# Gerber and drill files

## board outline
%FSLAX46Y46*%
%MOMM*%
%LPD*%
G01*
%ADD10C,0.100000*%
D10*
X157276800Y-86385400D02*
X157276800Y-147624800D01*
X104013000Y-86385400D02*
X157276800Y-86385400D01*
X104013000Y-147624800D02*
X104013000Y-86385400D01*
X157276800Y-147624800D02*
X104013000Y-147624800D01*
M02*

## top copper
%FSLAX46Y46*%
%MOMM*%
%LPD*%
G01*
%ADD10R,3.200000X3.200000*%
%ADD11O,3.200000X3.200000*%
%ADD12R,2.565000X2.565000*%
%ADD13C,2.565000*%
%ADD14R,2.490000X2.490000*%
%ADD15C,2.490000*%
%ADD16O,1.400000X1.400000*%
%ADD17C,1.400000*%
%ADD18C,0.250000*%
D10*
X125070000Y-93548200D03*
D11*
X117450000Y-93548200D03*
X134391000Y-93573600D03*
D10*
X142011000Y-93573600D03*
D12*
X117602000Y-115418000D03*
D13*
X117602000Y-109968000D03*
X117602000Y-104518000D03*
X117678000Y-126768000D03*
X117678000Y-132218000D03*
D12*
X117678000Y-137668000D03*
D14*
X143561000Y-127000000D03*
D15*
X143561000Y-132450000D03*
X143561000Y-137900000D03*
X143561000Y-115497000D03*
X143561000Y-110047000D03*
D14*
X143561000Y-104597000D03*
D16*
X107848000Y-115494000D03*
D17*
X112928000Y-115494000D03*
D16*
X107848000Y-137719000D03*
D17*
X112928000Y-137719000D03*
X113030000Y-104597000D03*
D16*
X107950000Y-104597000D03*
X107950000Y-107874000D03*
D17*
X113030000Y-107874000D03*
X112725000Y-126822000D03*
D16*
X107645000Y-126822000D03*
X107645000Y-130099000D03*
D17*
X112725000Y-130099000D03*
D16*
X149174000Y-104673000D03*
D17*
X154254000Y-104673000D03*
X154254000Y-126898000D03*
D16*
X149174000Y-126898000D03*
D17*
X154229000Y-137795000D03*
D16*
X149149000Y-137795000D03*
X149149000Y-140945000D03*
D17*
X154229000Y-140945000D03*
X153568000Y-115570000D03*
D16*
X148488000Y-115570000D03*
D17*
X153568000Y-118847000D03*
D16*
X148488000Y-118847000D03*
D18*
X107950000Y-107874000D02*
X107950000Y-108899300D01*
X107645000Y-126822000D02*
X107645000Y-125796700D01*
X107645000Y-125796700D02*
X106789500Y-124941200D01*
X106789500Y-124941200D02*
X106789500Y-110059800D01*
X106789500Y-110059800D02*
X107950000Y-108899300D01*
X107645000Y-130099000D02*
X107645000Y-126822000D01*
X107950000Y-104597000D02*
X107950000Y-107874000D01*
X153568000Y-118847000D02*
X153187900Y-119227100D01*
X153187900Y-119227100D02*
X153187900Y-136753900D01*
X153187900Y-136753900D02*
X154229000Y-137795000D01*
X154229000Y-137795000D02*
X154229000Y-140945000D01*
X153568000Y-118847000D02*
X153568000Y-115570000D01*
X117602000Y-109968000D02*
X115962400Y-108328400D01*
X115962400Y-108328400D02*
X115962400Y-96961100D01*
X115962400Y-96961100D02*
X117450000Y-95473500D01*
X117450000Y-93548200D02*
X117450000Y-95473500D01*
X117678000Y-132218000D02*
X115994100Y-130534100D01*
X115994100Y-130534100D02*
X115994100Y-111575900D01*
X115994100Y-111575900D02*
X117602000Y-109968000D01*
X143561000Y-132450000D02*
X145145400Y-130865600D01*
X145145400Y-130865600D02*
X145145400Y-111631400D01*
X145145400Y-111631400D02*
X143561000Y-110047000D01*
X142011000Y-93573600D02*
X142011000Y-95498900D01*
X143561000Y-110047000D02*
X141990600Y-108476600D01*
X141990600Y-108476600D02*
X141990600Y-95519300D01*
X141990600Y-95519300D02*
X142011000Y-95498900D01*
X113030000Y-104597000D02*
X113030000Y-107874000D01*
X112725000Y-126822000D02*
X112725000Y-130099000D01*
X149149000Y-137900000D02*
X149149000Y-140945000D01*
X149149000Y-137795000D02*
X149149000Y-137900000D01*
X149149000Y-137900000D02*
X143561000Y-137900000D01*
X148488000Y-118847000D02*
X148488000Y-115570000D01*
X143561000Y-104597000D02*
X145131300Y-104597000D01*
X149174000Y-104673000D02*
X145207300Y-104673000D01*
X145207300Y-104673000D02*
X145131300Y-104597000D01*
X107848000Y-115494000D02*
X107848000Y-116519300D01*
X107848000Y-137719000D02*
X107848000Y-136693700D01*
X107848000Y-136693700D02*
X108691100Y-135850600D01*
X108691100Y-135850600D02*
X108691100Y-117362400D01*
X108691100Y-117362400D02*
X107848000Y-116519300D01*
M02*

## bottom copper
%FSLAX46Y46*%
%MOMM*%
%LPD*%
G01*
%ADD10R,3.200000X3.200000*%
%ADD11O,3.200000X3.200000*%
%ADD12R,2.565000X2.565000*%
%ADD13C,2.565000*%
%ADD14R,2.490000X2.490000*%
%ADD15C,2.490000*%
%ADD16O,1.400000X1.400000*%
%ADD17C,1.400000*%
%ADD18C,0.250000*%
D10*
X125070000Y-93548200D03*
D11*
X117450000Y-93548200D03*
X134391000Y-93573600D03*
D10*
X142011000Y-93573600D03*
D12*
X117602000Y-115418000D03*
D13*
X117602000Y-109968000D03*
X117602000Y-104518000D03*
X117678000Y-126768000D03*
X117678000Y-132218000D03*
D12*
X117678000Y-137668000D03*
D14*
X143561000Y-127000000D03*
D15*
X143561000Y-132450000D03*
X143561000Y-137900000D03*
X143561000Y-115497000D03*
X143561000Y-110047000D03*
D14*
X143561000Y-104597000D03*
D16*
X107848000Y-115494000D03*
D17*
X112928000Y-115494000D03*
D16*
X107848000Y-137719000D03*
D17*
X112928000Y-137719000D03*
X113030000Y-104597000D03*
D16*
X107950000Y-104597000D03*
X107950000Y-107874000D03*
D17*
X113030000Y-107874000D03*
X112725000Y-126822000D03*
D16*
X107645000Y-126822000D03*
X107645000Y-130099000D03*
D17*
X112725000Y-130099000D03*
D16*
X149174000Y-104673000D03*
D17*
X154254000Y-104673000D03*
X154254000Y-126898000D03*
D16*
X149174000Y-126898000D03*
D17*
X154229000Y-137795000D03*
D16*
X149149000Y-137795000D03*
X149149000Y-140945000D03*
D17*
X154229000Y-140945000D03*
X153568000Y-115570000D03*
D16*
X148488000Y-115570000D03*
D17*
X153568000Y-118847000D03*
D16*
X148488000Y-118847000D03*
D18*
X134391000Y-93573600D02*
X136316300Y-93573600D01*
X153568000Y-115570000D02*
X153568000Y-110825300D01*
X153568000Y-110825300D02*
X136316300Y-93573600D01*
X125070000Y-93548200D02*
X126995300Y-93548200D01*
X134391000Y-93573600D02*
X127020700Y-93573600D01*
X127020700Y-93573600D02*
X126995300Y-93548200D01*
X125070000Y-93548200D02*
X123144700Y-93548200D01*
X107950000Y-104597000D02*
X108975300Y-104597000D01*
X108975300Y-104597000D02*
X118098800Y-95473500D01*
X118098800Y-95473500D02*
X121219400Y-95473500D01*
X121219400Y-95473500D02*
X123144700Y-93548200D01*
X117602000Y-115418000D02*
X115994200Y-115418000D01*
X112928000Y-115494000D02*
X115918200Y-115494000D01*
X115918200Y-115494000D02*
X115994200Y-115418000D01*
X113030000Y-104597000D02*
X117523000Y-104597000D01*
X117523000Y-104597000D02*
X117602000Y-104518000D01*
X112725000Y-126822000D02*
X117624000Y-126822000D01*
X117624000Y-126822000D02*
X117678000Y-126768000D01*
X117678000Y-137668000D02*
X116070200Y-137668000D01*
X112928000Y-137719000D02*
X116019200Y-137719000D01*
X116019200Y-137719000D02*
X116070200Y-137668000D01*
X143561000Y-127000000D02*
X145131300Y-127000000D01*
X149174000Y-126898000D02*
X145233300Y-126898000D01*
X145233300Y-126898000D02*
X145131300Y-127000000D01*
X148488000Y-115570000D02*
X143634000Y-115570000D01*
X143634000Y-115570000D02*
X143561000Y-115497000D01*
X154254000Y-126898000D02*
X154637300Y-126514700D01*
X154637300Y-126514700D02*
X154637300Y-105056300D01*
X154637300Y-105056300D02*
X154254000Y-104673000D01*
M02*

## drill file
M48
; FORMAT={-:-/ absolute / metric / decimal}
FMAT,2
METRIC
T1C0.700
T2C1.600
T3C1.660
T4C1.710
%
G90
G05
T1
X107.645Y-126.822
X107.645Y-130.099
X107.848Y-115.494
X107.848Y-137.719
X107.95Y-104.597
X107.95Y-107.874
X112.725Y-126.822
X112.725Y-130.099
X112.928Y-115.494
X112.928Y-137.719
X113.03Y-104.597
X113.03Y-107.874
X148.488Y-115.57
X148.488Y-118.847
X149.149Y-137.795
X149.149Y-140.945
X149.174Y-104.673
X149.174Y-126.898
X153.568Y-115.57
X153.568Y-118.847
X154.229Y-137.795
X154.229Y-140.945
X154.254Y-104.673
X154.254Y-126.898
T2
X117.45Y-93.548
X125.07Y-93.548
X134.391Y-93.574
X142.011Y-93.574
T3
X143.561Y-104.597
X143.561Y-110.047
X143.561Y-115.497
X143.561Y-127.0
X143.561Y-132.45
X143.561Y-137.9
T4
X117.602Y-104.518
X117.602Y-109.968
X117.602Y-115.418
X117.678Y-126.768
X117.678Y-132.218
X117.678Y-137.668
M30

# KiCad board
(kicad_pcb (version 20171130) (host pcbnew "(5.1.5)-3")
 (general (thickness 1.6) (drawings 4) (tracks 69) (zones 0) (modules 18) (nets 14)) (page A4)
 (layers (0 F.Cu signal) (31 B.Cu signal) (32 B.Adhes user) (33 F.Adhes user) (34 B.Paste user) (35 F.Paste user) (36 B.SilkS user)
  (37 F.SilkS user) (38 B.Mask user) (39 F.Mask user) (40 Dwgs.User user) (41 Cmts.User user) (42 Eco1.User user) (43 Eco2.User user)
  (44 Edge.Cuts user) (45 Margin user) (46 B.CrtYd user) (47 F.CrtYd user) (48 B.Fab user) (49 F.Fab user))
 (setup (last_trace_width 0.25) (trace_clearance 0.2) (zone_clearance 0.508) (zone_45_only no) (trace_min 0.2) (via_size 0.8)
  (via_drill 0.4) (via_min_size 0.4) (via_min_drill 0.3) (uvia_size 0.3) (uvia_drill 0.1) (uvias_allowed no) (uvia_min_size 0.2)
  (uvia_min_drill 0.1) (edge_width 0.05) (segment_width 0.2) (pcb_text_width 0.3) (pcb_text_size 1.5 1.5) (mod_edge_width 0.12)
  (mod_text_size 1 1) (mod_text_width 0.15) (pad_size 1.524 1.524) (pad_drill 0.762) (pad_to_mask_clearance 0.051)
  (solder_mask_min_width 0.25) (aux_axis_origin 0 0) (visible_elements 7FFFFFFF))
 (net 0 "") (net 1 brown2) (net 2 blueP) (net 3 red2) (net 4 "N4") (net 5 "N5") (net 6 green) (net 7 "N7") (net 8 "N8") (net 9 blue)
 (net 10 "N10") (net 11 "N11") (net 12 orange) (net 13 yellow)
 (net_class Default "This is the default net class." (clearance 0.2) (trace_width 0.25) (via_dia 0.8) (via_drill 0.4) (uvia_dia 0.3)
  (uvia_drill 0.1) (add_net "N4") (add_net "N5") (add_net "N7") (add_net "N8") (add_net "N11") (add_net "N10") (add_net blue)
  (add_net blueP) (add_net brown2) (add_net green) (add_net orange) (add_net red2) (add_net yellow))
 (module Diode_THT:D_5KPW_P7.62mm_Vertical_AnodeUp (layer F.Cu) (at 125.07 93.5482 180)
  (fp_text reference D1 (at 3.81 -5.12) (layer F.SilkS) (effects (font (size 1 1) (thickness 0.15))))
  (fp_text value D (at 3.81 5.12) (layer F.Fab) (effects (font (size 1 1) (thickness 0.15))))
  (pad 1 thru_hole rect (at 0 0 180) (size 3.2 3.2) (drill 1.6) (layers *.Cu *.Mask) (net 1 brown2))
  (pad 2 thru_hole oval (at 7.62 0 180) (size 3.2 3.2) (drill 1.6) (layers *.Cu *.Mask) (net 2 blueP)))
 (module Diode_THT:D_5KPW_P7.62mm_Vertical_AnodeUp (layer F.Cu) (at 142.011 93.5736 180)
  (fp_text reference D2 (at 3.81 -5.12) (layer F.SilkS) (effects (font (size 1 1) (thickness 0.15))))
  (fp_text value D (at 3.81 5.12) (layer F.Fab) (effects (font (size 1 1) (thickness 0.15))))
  (pad 2 thru_hole oval (at 7.62 0 180) (size 3.2 3.2) (drill 1.6) (layers *.Cu *.Mask) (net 1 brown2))
  (pad 1 thru_hole rect (at 0 0 180) (size 3.2 3.2) (drill 1.6) (layers *.Cu *.Mask) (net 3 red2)))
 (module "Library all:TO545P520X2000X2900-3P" (layer B.Cu) (at 117.602 115.418 90)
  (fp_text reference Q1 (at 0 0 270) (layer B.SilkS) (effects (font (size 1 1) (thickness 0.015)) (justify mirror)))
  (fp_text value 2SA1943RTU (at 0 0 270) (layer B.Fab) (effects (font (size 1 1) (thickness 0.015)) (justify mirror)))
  (pad 1 thru_hole rect (at 0 0 90) (size 2.565 2.565) (drill 1.71) (layers *.Cu *.Mask) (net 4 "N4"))
  (pad 2 thru_hole circle (at 5.45 0 90) (size 2.565 2.565) (drill 1.71) (layers *.Cu *.Mask) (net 2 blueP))
  (pad 3 thru_hole circle (at 10.9 0 90) (size 2.565 2.565) (drill 1.71) (layers *.Cu *.Mask) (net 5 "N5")))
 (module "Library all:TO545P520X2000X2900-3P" (layer B.Cu) (at 117.678 137.668 90)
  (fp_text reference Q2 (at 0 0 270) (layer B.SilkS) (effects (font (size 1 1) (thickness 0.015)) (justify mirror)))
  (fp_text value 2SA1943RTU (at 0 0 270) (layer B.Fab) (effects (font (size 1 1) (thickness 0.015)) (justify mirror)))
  (pad 3 thru_hole circle (at 10.9 0 90) (size 2.565 2.565) (drill 1.71) (layers *.Cu *.Mask) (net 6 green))
  (pad 2 thru_hole circle (at 5.45 0 90) (size 2.565 2.565) (drill 1.71) (layers *.Cu *.Mask) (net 2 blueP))
  (pad 1 thru_hole rect (at 0 0 90) (size 2.565 2.565) (drill 1.71) (layers *.Cu *.Mask) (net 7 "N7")))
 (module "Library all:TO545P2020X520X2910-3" (layer B.Cu) (at 143.561 127 270)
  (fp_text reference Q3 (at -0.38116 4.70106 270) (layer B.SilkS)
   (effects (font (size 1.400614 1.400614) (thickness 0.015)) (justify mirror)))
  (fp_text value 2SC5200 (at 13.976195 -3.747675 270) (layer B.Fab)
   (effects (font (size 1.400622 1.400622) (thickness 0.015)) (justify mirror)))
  (pad 1 thru_hole rect (at 0 0 270) (size 2.49 2.49) (drill 1.66) (layers *.Cu *.Mask) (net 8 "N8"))
  (pad 2 thru_hole circle (at 5.45 0 270) (size 2.49 2.49) (drill 1.66) (layers *.Cu *.Mask) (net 3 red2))
  (pad 3 thru_hole circle (at 10.9 0 270) (size 2.49 2.49) (drill 1.66) (layers *.Cu *.Mask) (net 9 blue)))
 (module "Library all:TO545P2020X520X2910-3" (layer B.Cu) (at 143.561 104.597 270)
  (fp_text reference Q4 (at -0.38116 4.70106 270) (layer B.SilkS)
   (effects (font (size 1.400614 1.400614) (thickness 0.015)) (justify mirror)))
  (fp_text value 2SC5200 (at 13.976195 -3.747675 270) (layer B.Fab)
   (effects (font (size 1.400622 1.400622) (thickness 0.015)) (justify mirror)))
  (pad 3 thru_hole circle (at 10.9 0 270) (size 2.49 2.49) (drill 1.66) (layers *.Cu *.Mask) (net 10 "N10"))
  (pad 2 thru_hole circle (at 5.45 0 270) (size 2.49 2.49) (drill 1.66) (layers *.Cu *.Mask) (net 3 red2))
  (pad 1 thru_hole rect (at 0 0 270) (size 2.49 2.49) (drill 1.66) (layers *.Cu *.Mask) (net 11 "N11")))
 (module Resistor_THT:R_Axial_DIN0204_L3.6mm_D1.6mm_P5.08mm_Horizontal (layer F.Cu) (at 112.928 115.494 180)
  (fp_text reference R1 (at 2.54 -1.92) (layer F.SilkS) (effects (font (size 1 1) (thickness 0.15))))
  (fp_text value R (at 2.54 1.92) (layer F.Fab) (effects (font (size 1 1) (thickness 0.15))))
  (pad 2 thru_hole oval (at 5.08 0 180) (size 1.4 1.4) (drill 0.7) (layers *.Cu *.Mask) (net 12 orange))
  (pad 1 thru_hole circle (at 0 0 180) (size 1.4 1.4) (drill 0.7) (layers *.Cu *.Mask) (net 4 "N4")))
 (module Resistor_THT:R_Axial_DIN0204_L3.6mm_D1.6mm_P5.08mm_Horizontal (layer F.Cu) (at 112.928 137.719 180)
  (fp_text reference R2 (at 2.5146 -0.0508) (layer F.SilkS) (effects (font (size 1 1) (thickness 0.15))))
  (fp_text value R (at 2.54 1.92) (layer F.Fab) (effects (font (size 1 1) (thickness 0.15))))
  (pad 2 thru_hole oval (at 5.08 0 180) (size 1.4 1.4) (drill 0.7) (layers *.Cu *.Mask) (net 12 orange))
  (pad 1 thru_hole circle (at 0 0 180) (size 1.4 1.4) (drill 0.7) (layers *.Cu *.Mask) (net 7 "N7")))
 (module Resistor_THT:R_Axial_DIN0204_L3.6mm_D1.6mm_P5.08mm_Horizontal (layer F.Cu) (at 113.03 104.597 180)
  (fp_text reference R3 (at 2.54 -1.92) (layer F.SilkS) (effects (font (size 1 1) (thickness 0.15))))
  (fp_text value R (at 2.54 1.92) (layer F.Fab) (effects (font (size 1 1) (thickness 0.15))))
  (pad 1 thru_hole circle (at 0 0 180) (size 1.4 1.4) (drill 0.7) (layers *.Cu *.Mask) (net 5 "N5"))
  (pad 2 thru_hole oval (at 5.08 0 180) (size 1.4 1.4) (drill 0.7) (layers *.Cu *.Mask) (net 1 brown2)))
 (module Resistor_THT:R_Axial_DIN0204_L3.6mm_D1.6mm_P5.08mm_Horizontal (layer F.Cu) (at 113.03 107.874 180)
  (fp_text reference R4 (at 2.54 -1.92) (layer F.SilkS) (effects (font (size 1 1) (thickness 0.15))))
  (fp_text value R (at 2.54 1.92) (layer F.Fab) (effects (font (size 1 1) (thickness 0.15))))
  (pad 2 thru_hole oval (at 5.08 0 180) (size 1.4 1.4) (drill 0.7) (layers *.Cu *.Mask) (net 1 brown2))
  (pad 1 thru_hole circle (at 0 0 180) (size 1.4 1.4) (drill 0.7) (layers *.Cu *.Mask) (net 5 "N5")))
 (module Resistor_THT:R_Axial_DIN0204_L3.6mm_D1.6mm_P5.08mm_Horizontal (layer F.Cu) (at 112.725 126.822 180)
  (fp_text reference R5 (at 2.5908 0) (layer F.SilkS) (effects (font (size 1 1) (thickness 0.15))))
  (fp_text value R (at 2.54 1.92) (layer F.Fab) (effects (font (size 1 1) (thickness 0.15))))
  (pad 1 thru_hole circle (at 0 0 180) (size 1.4 1.4) (drill 0.7) (layers *.Cu *.Mask) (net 6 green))
  (pad 2 thru_hole oval (at 5.08 0 180) (size 1.4 1.4) (drill 0.7) (layers *.Cu *.Mask) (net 1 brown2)))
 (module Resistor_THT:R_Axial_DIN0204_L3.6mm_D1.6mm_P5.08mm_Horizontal (layer F.Cu) (at 112.725 130.099 180)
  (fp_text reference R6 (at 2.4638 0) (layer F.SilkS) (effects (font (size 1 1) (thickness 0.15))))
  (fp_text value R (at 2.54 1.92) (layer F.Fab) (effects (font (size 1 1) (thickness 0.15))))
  (pad 2 thru_hole oval (at 5.08 0 180) (size 1.4 1.4) (drill 0.7) (layers *.Cu *.Mask) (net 1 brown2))
  (pad 1 thru_hole circle (at 0 0 180) (size 1.4 1.4) (drill 0.7) (layers *.Cu *.Mask) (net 6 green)))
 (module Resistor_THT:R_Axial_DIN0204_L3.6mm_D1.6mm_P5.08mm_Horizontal (layer F.Cu) (at 154.254 104.673 180)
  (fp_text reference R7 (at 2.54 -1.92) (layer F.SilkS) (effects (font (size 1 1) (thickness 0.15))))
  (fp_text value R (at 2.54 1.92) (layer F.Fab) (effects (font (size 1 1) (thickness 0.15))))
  (pad 2 thru_hole oval (at 5.08 0 180) (size 1.4 1.4) (drill 0.7) (layers *.Cu *.Mask) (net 11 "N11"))
  (pad 1 thru_hole circle (at 0 0 180) (size 1.4 1.4) (drill 0.7) (layers *.Cu *.Mask) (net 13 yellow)))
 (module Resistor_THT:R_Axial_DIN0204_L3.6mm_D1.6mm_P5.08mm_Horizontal (layer F.Cu) (at 154.254 126.898 180)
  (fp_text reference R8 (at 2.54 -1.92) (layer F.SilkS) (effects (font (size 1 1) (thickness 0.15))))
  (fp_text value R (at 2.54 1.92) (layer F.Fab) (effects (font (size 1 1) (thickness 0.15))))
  (pad 1 thru_hole circle (at 0 0 180) (size 1.4 1.4) (drill 0.7) (layers *.Cu *.Mask) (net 13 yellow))
  (pad 2 thru_hole oval (at 5.08 0 180) (size 1.4 1.4) (drill 0.7) (layers *.Cu *.Mask) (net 8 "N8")))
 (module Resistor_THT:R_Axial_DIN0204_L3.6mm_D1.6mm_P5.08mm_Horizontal (layer F.Cu) (at 154.229 137.795 180)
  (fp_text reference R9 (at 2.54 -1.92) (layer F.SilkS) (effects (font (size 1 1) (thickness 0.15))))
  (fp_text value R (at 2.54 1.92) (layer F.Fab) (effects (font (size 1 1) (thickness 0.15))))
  (pad 1 thru_hole circle (at 0 0 180) (size 1.4 1.4) (drill 0.7) (layers *.Cu *.Mask) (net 1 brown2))
  (pad 2 thru_hole oval (at 5.08 0 180) (size 1.4 1.4) (drill 0.7) (layers *.Cu *.Mask) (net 9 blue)))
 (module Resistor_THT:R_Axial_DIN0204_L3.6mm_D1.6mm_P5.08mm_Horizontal (layer F.Cu) (at 154.229 140.945 180)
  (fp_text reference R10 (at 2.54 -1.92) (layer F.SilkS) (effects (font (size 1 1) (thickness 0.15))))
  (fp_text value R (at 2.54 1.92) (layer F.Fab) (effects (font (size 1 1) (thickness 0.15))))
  (pad 2 thru_hole oval (at 5.08 0 180) (size 1.4 1.4) (drill 0.7) (layers *.Cu *.Mask) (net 9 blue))
  (pad 1 thru_hole circle (at 0 0 180) (size 1.4 1.4) (drill 0.7) (layers *.Cu *.Mask) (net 1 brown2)))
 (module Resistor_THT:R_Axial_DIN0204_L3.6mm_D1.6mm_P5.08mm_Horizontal (layer F.Cu) (at 153.568 115.57 180)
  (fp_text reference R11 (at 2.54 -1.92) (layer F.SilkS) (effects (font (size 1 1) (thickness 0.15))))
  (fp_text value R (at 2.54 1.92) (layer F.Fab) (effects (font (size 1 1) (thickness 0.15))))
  (pad 1 thru_hole circle (at 0 0 180) (size 1.4 1.4) (drill 0.7) (layers *.Cu *.Mask) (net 1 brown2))
  (pad 2 thru_hole oval (at 5.08 0 180) (size 1.4 1.4) (drill 0.7) (layers *.Cu *.Mask) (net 10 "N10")))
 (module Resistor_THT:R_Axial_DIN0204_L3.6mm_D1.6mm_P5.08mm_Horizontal (layer F.Cu) (at 153.568 118.847 180)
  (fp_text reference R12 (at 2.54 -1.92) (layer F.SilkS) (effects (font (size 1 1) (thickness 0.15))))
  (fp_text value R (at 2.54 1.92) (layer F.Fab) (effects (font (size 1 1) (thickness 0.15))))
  (pad 1 thru_hole circle (at 0 0 180) (size 1.4 1.4) (drill 0.7) (layers *.Cu *.Mask) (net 1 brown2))
  (pad 2 thru_hole oval (at 5.08 0 180) (size 1.4 1.4) (drill 0.7) (layers *.Cu *.Mask) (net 10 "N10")))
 (gr_line (start 157.2768 86.3854) (end 157.2768 147.6248) (layer Edge.Cuts) (width 0.1))
 (gr_line (start 104.013 86.3854) (end 157.2768 86.3854) (layer Edge.Cuts) (width 0.1))
 (gr_line (start 104.013 147.6248) (end 104.013 86.3854) (layer Edge.Cuts) (width 0.1))
 (gr_line (start 157.2768 147.6248) (end 104.013 147.6248) (layer Edge.Cuts) (width 0.1))
 (segment (start 134.391 93.5736) (end 136.3163 93.5736) (width 0.25) (layer B.Cu) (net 1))
 (segment (start 153.568 115.57) (end 153.568 110.8253) (width 0.25) (layer B.Cu) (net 1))
 (segment (start 153.568 110.8253) (end 136.3163 93.5736) (width 0.25) (layer B.Cu) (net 1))
 (segment (start 125.07 93.5482) (end 126.9953 93.5482) (width 0.25) (layer B.Cu) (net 1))
 (segment (start 134.391 93.5736) (end 127.0207 93.5736) (width 0.25) (layer B.Cu) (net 1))
 (segment (start 127.0207 93.5736) (end 126.9953 93.5482) (width 0.25) (layer B.Cu) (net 1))
 (segment (start 125.07 93.5482) (end 123.1447 93.5482) (width 0.25) (layer B.Cu) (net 1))
 (segment (start 107.95 104.597) (end 108.9753 104.597) (width 0.25) (layer B.Cu) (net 1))
 (segment (start 108.9753 104.597) (end 118.0988 95.4735) (width 0.25) (layer B.Cu) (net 1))
 (segment (start 118.0988 95.4735) (end 121.2194 95.4735) (width 0.25) (layer B.Cu) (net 1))
 (segment (start 121.2194 95.4735) (end 123.1447 93.5482) (width 0.25) (layer B.Cu) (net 1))
 (segment (start 107.95 107.874) (end 107.95 108.8993) (width 0.25) (layer F.Cu) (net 1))
 (segment (start 107.645 126.822) (end 107.645 125.7967) (width 0.25) (layer F.Cu) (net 1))
 (segment (start 107.645 125.7967) (end 106.7895 124.9412) (width 0.25) (layer F.Cu) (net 1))
 (segment (start 106.7895 124.9412) (end 106.7895 110.0598) (width 0.25) (layer F.Cu) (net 1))
 (segment (start 106.7895 110.0598) (end 107.95 108.8993) (width 0.25) (layer F.Cu) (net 1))
 (segment (start 107.645 130.099) (end 107.645 126.822) (width 0.25) (layer F.Cu) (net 1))
 (segment (start 107.95 104.597) (end 107.95 107.874) (width 0.25) (layer F.Cu) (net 1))
 (segment (start 153.568 118.847) (end 153.1879 119.2271) (width 0.25) (layer F.Cu) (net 1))
 (segment (start 153.1879 119.2271) (end 153.1879 136.7539) (width 0.25) (layer F.Cu) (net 1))
 (segment (start 153.1879 136.7539) (end 154.229 137.795) (width 0.25) (layer F.Cu) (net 1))
 (segment (start 154.229 137.795) (end 154.229 140.945) (width 0.25) (layer F.Cu) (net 1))
 (segment (start 153.568 118.847) (end 153.568 115.57) (width 0.25) (layer F.Cu) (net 1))
 (segment (start 117.602 109.968) (end 115.9624 108.3284) (width 0.25) (layer F.Cu) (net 2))
 (segment (start 115.9624 108.3284) (end 115.9624 96.9611) (width 0.25) (layer F.Cu) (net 2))
 (segment (start 115.9624 96.9611) (end 117.45 95.4735) (width 0.25) (layer F.Cu) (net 2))
 (segment (start 117.45 93.5482) (end 117.45 95.4735) (width 0.25) (layer F.Cu) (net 2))
 (segment (start 117.678 132.218) (end 115.9941 130.5341) (width 0.25) (layer F.Cu) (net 2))
 (segment (start 115.9941 130.5341) (end 115.9941 111.5759) (width 0.25) (layer F.Cu) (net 2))
 (segment (start 115.9941 111.5759) (end 117.602 109.968) (width 0.25) (layer F.Cu) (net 2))
 (segment (start 143.561 132.45) (end 145.1454 130.8656) (width 0.25) (layer F.Cu) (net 3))
 (segment (start 145.1454 130.8656) (end 145.1454 111.6314) (width 0.25) (layer F.Cu) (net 3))
 (segment (start 145.1454 111.6314) (end 143.561 110.047) (width 0.25) (layer F.Cu) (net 3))
 (segment (start 142.011 93.5736) (end 142.011 95.4989) (width 0.25) (layer F.Cu) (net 3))
 (segment (start 143.561 110.047) (end 141.9906 108.4766) (width 0.25) (layer F.Cu) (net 3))
 (segment (start 141.9906 108.4766) (end 141.9906 95.5193) (width 0.25) (layer F.Cu) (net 3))
 (segment (start 141.9906 95.5193) (end 142.011 95.4989) (width 0.25) (layer F.Cu) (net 3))
 (segment (start 117.602 115.418) (end 115.9942 115.418) (width 0.25) (layer B.Cu) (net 4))
 (segment (start 112.928 115.494) (end 115.9182 115.494) (width 0.25) (layer B.Cu) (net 4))
 (segment (start 115.9182 115.494) (end 115.9942 115.418) (width 0.25) (layer B.Cu) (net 4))
 (segment (start 113.03 104.597) (end 117.523 104.597) (width 0.25) (layer B.Cu) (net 5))
 (segment (start 117.523 104.597) (end 117.602 104.518) (width 0.25) (layer B.Cu) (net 5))
 (segment (start 113.03 104.597) (end 113.03 107.874) (width 0.25) (layer F.Cu) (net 5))
 (segment (start 112.725 126.822) (end 117.624 126.822) (width 0.25) (layer B.Cu) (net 6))
 (segment (start 117.624 126.822) (end 117.678 126.768) (width 0.25) (layer B.Cu) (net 6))
 (segment (start 112.725 126.822) (end 112.725 130.099) (width 0.25) (layer F.Cu) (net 6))
 (segment (start 117.678 137.668) (end 116.0702 137.668) (width 0.25) (layer B.Cu) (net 7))
 (segment (start 112.928 137.719) (end 116.0192 137.719) (width 0.25) (layer B.Cu) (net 7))
 (segment (start 116.0192 137.719) (end 116.0702 137.668) (width 0.25) (layer B.Cu) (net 7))
 (segment (start 143.561 127) (end 145.1313 127) (width 0.25) (layer B.Cu) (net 8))
 (segment (start 149.174 126.898) (end 145.2333 126.898) (width 0.25) (layer B.Cu) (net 8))
 (segment (start 145.2333 126.898) (end 145.1313 127) (width 0.25) (layer B.Cu) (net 8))
 (segment (start 149.149 137.9) (end 149.149 140.945) (width 0.25) (layer F.Cu) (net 9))
 (segment (start 149.149 137.795) (end 149.149 137.9) (width 0.25) (layer F.Cu) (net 9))
 (segment (start 149.149 137.9) (end 143.561 137.9) (width 0.25) (layer F.Cu) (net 9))
 (segment (start 148.488 115.57) (end 143.634 115.57) (width 0.25) (layer B.Cu) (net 10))
 (segment (start 143.634 115.57) (end 143.561 115.497) (width 0.25) (layer B.Cu) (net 10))
 (segment (start 148.488 118.847) (end 148.488 115.57) (width 0.25) (layer F.Cu) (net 10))
 (segment (start 143.561 104.597) (end 145.1313 104.597) (width 0.25) (layer F.Cu) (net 11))
 (segment (start 149.174 104.673) (end 145.2073 104.673) (width 0.25) (layer F.Cu) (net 11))
 (segment (start 145.2073 104.673) (end 145.1313 104.597) (width 0.25) (layer F.Cu) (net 11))
 (segment (start 107.848 115.494) (end 107.848 116.5193) (width 0.25) (layer F.Cu) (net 12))
 (segment (start 107.848 137.719) (end 107.848 136.6937) (width 0.25) (layer F.Cu) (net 12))
 (segment (start 107.848 136.6937) (end 108.6911 135.8506) (width 0.25) (layer F.Cu) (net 12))
 (segment (start 108.6911 135.8506) (end 108.6911 117.3624) (width 0.25) (layer F.Cu) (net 12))
 (segment (start 108.6911 117.3624) (end 107.848 116.5193) (width 0.25) (layer F.Cu) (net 12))
 (segment (start 154.254 126.898) (end 154.6373 126.5147) (width 0.25) (layer B.Cu) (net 13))
 (segment (start 154.6373 126.5147) (end 154.6373 105.0563) (width 0.25) (layer B.Cu) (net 13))
 (segment (start 154.6373 105.0563) (end 154.254 104.673) (width 0.25) (layer B.Cu) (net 13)))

